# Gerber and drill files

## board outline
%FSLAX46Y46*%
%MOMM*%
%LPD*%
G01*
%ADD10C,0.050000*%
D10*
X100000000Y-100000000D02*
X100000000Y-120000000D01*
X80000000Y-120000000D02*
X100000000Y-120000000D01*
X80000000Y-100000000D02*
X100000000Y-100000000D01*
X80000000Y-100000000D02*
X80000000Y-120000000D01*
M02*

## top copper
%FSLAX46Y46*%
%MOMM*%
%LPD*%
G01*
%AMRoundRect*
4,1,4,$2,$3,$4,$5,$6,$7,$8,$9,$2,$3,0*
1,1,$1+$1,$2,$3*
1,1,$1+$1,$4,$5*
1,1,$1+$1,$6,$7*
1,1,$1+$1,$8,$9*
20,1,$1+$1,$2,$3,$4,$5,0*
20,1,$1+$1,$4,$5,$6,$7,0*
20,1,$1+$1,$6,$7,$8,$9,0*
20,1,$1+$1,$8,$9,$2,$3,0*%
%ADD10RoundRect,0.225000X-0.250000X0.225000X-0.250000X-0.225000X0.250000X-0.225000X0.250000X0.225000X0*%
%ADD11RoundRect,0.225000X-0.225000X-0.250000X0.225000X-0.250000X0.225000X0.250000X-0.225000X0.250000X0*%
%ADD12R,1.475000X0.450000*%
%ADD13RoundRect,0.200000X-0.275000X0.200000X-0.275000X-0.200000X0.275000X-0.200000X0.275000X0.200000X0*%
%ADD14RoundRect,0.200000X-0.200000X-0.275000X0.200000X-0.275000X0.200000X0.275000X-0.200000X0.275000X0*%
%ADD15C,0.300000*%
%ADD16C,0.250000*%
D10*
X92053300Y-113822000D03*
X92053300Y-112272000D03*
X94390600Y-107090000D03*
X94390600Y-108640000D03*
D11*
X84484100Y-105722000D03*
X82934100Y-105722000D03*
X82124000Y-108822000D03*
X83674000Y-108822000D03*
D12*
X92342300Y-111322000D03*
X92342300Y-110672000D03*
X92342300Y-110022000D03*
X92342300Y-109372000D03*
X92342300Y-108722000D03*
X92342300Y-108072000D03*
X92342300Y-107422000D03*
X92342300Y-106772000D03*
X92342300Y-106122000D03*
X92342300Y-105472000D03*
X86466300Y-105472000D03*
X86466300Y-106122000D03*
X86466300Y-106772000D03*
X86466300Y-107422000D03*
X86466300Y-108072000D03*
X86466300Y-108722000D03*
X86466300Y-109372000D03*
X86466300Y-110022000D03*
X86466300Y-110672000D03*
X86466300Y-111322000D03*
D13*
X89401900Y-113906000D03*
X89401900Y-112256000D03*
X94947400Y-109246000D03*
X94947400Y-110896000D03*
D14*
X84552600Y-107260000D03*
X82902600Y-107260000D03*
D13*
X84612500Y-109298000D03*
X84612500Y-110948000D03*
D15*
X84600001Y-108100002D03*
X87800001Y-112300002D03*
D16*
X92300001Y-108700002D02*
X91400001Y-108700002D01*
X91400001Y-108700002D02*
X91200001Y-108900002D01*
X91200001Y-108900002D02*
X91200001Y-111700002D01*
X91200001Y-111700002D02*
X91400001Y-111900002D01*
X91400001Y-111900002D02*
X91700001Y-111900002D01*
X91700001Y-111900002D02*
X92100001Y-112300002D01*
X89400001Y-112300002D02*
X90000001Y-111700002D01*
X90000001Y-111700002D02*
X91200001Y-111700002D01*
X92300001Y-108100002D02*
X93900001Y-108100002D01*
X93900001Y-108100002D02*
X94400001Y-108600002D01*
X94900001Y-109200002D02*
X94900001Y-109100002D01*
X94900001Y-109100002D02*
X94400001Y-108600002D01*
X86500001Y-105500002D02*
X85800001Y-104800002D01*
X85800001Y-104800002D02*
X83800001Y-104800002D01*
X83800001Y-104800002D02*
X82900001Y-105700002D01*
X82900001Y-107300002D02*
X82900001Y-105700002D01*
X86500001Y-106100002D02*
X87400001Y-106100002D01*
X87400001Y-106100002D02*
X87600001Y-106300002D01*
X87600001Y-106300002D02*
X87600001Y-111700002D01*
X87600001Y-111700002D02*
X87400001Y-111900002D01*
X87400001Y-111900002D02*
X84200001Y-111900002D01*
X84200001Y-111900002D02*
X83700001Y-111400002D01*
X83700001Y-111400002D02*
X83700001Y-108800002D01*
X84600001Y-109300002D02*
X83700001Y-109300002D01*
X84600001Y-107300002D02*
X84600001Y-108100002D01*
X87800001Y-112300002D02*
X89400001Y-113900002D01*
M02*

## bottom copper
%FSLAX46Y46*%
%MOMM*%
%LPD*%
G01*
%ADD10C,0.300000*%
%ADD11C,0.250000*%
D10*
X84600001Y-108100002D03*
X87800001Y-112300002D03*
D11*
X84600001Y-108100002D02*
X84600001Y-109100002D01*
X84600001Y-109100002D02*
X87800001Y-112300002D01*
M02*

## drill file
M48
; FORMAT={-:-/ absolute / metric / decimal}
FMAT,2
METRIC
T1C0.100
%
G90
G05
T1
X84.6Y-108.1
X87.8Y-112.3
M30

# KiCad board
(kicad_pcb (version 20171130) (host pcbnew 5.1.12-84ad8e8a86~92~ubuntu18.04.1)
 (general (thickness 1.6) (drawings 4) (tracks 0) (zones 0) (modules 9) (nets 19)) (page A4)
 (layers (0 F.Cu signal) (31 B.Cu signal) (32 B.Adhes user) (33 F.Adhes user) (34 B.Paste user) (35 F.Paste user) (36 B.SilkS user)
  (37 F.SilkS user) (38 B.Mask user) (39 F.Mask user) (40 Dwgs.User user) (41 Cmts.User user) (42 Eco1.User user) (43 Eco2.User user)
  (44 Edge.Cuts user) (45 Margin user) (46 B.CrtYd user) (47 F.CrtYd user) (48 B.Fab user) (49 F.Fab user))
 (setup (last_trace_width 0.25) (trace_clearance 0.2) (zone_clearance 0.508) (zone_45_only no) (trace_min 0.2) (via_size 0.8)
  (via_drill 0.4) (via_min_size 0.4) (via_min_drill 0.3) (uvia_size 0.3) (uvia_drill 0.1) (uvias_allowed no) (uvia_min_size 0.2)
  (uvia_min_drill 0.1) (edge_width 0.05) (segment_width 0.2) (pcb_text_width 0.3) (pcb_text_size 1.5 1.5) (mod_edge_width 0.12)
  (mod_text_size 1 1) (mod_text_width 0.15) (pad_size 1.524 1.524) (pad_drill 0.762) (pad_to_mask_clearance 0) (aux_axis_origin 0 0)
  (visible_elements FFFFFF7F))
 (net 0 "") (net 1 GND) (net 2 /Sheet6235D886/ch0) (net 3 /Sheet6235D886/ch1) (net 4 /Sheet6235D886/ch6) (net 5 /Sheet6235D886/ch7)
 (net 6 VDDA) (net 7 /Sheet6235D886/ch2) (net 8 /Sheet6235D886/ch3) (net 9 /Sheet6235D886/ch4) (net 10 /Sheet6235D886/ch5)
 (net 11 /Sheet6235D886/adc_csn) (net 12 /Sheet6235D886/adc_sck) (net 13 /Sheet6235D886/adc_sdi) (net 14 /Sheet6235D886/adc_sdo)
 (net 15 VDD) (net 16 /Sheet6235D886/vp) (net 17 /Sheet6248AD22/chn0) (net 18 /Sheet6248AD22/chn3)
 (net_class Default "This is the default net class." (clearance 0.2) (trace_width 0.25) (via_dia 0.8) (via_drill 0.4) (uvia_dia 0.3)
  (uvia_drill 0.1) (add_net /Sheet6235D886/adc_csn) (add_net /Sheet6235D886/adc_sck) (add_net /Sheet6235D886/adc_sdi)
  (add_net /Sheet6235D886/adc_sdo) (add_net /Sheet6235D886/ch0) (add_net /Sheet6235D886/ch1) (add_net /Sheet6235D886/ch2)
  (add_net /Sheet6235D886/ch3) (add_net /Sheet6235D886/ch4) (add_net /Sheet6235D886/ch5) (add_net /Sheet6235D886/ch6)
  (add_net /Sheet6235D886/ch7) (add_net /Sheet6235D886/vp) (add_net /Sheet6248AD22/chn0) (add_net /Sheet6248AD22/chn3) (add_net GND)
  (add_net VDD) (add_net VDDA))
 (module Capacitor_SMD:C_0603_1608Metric (layer F.Cu) (at 92.053300 113.047000 270.000000)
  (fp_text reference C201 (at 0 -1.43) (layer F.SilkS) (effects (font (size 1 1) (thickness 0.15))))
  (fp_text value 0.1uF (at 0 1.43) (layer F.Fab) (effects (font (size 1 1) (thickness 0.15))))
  (pad 2 smd roundrect (at 0.775 0 270.000000) (size 0.9 0.95) (layers F.Cu F.Mask F.Paste) (roundrect_rratio 0.25) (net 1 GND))
  (pad 1 smd roundrect (at -0.775 0 270.000000) (size 0.9 0.95) (layers F.Cu F.Mask F.Paste) (roundrect_rratio 0.25)
   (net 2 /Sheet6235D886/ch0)))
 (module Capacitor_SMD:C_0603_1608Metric (layer F.Cu) (at 94.390600 107.865000 270.000000)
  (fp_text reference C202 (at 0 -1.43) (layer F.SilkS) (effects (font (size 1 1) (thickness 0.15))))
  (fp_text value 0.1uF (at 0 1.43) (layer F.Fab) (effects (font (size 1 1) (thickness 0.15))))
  (pad 1 smd roundrect (at -0.775 0 270.000000) (size 0.9 0.95) (layers F.Cu F.Mask F.Paste) (roundrect_rratio 0.25) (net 1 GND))
  (pad 2 smd roundrect (at 0.775 0 270.000000) (size 0.9 0.95) (layers F.Cu F.Mask F.Paste) (roundrect_rratio 0.25)
   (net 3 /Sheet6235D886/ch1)))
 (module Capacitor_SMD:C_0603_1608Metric (layer F.Cu) (at 83.709100 105.722000)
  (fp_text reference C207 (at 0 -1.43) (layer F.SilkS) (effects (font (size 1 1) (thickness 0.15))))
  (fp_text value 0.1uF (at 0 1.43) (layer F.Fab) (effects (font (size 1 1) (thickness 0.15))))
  (pad 2 smd roundrect (at 0.775 0) (size 0.9 0.95) (layers F.Cu F.Mask F.Paste) (roundrect_rratio 0.25) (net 1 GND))
  (pad 1 smd roundrect (at -0.775 0) (size 0.9 0.95) (layers F.Cu F.Mask F.Paste) (roundrect_rratio 0.25) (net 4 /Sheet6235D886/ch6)))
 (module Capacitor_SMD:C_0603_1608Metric (layer F.Cu) (at 82.899000 108.822000)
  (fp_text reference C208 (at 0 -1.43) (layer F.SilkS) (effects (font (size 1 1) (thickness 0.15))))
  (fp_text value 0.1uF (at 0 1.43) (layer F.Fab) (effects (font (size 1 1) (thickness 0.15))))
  (pad 1 smd roundrect (at -0.775 0) (size 0.9 0.95) (layers F.Cu F.Mask F.Paste) (roundrect_rratio 0.25) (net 1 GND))
  (pad 2 smd roundrect (at 0.775 0) (size 0.9 0.95) (layers F.Cu F.Mask F.Paste) (roundrect_rratio 0.25) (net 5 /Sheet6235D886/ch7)))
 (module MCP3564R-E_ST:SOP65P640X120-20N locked (layer F.Cu) (at 89.404300 108.397000 180.000000)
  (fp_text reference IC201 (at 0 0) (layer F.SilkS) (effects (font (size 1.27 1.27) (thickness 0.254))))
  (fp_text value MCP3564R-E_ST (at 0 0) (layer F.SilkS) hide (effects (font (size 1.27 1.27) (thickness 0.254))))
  (pad 1 smd rect (at -2.938 -2.925 270.000000) (size 0.45 1.475) (layers F.Cu F.Mask F.Paste) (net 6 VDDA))
  (pad 2 smd rect (at -2.938 -2.275 270.000000) (size 0.45 1.475) (layers F.Cu F.Mask F.Paste) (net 1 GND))
  (pad 3 smd rect (at -2.938 -1.625 270.000000) (size 0.45 1.475) (layers F.Cu F.Mask F.Paste) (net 1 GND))
  (pad 4 smd rect (at -2.938 -0.975 270.000000) (size 0.45 1.475) (layers F.Cu F.Mask F.Paste))
  (pad 5 smd rect (at -2.938 -0.325 270.000000) (size 0.45 1.475) (layers F.Cu F.Mask F.Paste) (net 2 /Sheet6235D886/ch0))
  (pad 6 smd rect (at -2.938 0.325 270.000000) (size 0.45 1.475) (layers F.Cu F.Mask F.Paste) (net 3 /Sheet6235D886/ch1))
  (pad 7 smd rect (at -2.938 0.975 270.000000) (size 0.45 1.475) (layers F.Cu F.Mask F.Paste) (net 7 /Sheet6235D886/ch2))
  (pad 8 smd rect (at -2.938 1.625 270.000000) (size 0.45 1.475) (layers F.Cu F.Mask F.Paste) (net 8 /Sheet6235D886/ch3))
  (pad 9 smd rect (at -2.938 2.275 270.000000) (size 0.45 1.475) (layers F.Cu F.Mask F.Paste) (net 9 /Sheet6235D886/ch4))
  (pad 10 smd rect (at -2.938 2.925 270.000000) (size 0.45 1.475) (layers F.Cu F.Mask F.Paste) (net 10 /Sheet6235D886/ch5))
  (pad 11 smd rect (at 2.938 2.925 270.000000) (size 0.45 1.475) (layers F.Cu F.Mask F.Paste) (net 4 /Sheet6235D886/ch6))
  (pad 12 smd rect (at 2.938 2.275 270.000000) (size 0.45 1.475) (layers F.Cu F.Mask F.Paste) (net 5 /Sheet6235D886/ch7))
  (pad 13 smd rect (at 2.938 1.625 270.000000) (size 0.45 1.475) (layers F.Cu F.Mask F.Paste) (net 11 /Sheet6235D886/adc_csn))
  (pad 14 smd rect (at 2.938 0.975 270.000000) (size 0.45 1.475) (layers F.Cu F.Mask F.Paste) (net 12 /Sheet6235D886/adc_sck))
  (pad 15 smd rect (at 2.938 0.325 270.000000) (size 0.45 1.475) (layers F.Cu F.Mask F.Paste) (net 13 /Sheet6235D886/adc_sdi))
  (pad 16 smd rect (at 2.938 -0.325 270.000000) (size 0.45 1.475) (layers F.Cu F.Mask F.Paste) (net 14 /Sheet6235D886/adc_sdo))
  (pad 17 smd rect (at 2.938 -0.975 270.000000) (size 0.45 1.475) (layers F.Cu F.Mask F.Paste))
  (pad 18 smd rect (at 2.938 -1.625 270.000000) (size 0.45 1.475) (layers F.Cu F.Mask F.Paste))
  (pad 19 smd rect (at 2.938 -2.275 270.000000) (size 0.45 1.475) (layers F.Cu F.Mask F.Paste) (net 1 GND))
  (pad 20 smd rect (at 2.938 -2.925 270.000000) (size 0.45 1.475) (layers F.Cu F.Mask F.Paste) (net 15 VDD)))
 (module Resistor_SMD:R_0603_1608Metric (layer F.Cu) (at 89.401900 113.081000 270.000000)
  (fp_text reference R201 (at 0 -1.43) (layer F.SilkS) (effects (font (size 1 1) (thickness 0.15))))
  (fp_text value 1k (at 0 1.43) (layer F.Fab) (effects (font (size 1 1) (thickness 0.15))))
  (pad 2 smd roundrect (at 0.825 0 270.000000) (size 0.8 0.95) (layers F.Cu F.Mask F.Paste) (roundrect_rratio 0.25)
   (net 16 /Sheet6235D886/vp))
  (pad 1 smd roundrect (at -0.825 0 270.000000) (size 0.8 0.95) (layers F.Cu F.Mask F.Paste) (roundrect_rratio 0.25)
   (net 2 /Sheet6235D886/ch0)))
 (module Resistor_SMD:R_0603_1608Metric (layer F.Cu) (at 94.947400 110.071000 270.000000)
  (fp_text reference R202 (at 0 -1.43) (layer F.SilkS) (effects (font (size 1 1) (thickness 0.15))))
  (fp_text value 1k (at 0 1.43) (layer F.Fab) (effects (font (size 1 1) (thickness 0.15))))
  (pad 1 smd roundrect (at -0.825 0 270.000000) (size 0.8 0.95) (layers F.Cu F.Mask F.Paste) (roundrect_rratio 0.25)
   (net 3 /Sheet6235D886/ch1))
  (pad 2 smd roundrect (at 0.825 0 270.000000) (size 0.8 0.95) (layers F.Cu F.Mask F.Paste) (roundrect_rratio 0.25)
   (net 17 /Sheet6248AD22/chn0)))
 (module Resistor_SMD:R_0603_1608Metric (layer F.Cu) (at 83.727600 107.260000)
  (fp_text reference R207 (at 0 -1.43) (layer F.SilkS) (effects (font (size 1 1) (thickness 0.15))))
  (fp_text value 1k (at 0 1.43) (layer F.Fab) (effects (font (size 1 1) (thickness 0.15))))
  (pad 2 smd roundrect (at 0.825 0) (size 0.8 0.95) (layers F.Cu F.Mask F.Paste) (roundrect_rratio 0.25) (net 16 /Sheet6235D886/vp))
  (pad 1 smd roundrect (at -0.825 0) (size 0.8 0.95) (layers F.Cu F.Mask F.Paste) (roundrect_rratio 0.25) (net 4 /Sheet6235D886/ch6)))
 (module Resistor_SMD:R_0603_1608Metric (layer F.Cu) (at 84.612500 110.123000 270.000000)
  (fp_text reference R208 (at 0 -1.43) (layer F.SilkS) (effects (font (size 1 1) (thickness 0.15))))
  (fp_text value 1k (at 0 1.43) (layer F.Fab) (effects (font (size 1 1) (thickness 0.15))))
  (pad 1 smd roundrect (at -0.825 0 270.000000) (size 0.8 0.95) (layers F.Cu F.Mask F.Paste) (roundrect_rratio 0.25)
   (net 5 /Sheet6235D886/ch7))
  (pad 2 smd roundrect (at 0.825 0 270.000000) (size 0.8 0.95) (layers F.Cu F.Mask F.Paste) (roundrect_rratio 0.25)
   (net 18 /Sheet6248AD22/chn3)))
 (gr_line (start 100 100) (end 100 120) (layer Edge.Cuts) (width 0.05))
 (gr_line (start 80 120) (end 100 120) (layer Edge.Cuts) (width 0.05))
 (gr_line (start 80 100) (end 100 100) (layer Edge.Cuts) (width 0.05))
 (gr_line (start 80 100) (end 80 120) (layer Edge.Cuts) (width 0.05))
 (segment (start 92.300001 108.700002) (end 91.400001 108.700002) (width 0.250000) (layer F.Cu) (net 2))
 (segment (start 91.400001 108.700002) (end 91.200001 108.900002) (width 0.250000) (layer F.Cu) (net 2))
 (segment (start 91.200001 108.900002) (end 91.200001 111.700002) (width 0.250000) (layer F.Cu) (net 2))
 (segment (start 91.200001 111.700002) (end 91.400001 111.900002) (width 0.250000) (layer F.Cu) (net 2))
 (segment (start 91.400001 111.900002) (end 91.700001 111.900002) (width 0.250000) (layer F.Cu) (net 2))
 (segment (start 91.700001 111.900002) (end 92.100001 112.300002) (width 0.250000) (layer F.Cu) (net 2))
 (segment (start 89.400001 112.300002) (end 90.000001 111.700002) (width 0.250000) (layer F.Cu) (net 2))
 (segment (start 90.000001 111.700002) (end 91.200001 111.700002) (width 0.250000) (layer F.Cu) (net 2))
 (segment (start 92.300001 108.100002) (end 93.900001 108.100002) (width 0.250000) (layer F.Cu) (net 3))
 (segment (start 93.900001 108.100002) (end 94.400001 108.600002) (width 0.250000) (layer F.Cu) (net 3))
 (segment (start 94.900001 109.200002) (end 94.900001 109.100002) (width 0.250000) (layer F.Cu) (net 3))
 (segment (start 94.900001 109.100002) (end 94.400001 108.600002) (width 0.250000) (layer F.Cu) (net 3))
 (segment (start 86.500001 105.500002) (end 85.800001 104.800002) (width 0.250000) (layer F.Cu) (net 4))
 (segment (start 85.800001 104.800002) (end 83.800001 104.800002) (width 0.250000) (layer F.Cu) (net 4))
 (segment (start 83.800001 104.800002) (end 82.900001 105.700002) (width 0.250000) (layer F.Cu) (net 4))
 (segment (start 82.900001 107.300002) (end 82.900001 105.700002) (width 0.250000) (layer F.Cu) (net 4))
 (segment (start 86.500001 106.100002) (end 87.400001 106.100002) (width 0.250000) (layer F.Cu) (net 5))
 (segment (start 87.400001 106.100002) (end 87.600001 106.300002) (width 0.250000) (layer F.Cu) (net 5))
 (segment (start 87.600001 106.300002) (end 87.600001 111.700002) (width 0.250000) (layer F.Cu) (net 5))
 (segment (start 87.600001 111.700002) (end 87.400001 111.900002) (width 0.250000) (layer F.Cu) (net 5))
 (segment (start 87.400001 111.900002) (end 84.200001 111.900002) (width 0.250000) (layer F.Cu) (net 5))
 (segment (start 84.200001 111.900002) (end 83.700001 111.400002) (width 0.250000) (layer F.Cu) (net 5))
 (segment (start 83.700001 111.400002) (end 83.700001 108.800002) (width 0.250000) (layer F.Cu) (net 5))
 (segment (start 84.600001 109.300002) (end 83.700001 109.300002) (width 0.250000) (layer F.Cu) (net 5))
 (segment (start 84.600001 107.300002) (end 84.600001 108.100002) (width 0.250000) (layer F.Cu) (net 16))
 (segment (start 84.600001 108.100002) (end 84.600001 109.100002) (width 0.250000) (layer B.Cu) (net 16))
 (segment (start 84.600001 109.100002) (end 87.800001 112.300002) (width 0.250000) (layer B.Cu) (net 16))
 (segment (start 87.800001 112.300002) (end 89.400001 113.900002) (width 0.250000) (layer F.Cu) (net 16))
 (via micro (at 84.600001 108.100002) (size 0.300000) (drill 0.100000) (layers F.Cu B.Cu) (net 16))
 (via micro (at 87.800001 112.300002) (size 0.300000) (drill 0.100000) (layers F.Cu B.Cu) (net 16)))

